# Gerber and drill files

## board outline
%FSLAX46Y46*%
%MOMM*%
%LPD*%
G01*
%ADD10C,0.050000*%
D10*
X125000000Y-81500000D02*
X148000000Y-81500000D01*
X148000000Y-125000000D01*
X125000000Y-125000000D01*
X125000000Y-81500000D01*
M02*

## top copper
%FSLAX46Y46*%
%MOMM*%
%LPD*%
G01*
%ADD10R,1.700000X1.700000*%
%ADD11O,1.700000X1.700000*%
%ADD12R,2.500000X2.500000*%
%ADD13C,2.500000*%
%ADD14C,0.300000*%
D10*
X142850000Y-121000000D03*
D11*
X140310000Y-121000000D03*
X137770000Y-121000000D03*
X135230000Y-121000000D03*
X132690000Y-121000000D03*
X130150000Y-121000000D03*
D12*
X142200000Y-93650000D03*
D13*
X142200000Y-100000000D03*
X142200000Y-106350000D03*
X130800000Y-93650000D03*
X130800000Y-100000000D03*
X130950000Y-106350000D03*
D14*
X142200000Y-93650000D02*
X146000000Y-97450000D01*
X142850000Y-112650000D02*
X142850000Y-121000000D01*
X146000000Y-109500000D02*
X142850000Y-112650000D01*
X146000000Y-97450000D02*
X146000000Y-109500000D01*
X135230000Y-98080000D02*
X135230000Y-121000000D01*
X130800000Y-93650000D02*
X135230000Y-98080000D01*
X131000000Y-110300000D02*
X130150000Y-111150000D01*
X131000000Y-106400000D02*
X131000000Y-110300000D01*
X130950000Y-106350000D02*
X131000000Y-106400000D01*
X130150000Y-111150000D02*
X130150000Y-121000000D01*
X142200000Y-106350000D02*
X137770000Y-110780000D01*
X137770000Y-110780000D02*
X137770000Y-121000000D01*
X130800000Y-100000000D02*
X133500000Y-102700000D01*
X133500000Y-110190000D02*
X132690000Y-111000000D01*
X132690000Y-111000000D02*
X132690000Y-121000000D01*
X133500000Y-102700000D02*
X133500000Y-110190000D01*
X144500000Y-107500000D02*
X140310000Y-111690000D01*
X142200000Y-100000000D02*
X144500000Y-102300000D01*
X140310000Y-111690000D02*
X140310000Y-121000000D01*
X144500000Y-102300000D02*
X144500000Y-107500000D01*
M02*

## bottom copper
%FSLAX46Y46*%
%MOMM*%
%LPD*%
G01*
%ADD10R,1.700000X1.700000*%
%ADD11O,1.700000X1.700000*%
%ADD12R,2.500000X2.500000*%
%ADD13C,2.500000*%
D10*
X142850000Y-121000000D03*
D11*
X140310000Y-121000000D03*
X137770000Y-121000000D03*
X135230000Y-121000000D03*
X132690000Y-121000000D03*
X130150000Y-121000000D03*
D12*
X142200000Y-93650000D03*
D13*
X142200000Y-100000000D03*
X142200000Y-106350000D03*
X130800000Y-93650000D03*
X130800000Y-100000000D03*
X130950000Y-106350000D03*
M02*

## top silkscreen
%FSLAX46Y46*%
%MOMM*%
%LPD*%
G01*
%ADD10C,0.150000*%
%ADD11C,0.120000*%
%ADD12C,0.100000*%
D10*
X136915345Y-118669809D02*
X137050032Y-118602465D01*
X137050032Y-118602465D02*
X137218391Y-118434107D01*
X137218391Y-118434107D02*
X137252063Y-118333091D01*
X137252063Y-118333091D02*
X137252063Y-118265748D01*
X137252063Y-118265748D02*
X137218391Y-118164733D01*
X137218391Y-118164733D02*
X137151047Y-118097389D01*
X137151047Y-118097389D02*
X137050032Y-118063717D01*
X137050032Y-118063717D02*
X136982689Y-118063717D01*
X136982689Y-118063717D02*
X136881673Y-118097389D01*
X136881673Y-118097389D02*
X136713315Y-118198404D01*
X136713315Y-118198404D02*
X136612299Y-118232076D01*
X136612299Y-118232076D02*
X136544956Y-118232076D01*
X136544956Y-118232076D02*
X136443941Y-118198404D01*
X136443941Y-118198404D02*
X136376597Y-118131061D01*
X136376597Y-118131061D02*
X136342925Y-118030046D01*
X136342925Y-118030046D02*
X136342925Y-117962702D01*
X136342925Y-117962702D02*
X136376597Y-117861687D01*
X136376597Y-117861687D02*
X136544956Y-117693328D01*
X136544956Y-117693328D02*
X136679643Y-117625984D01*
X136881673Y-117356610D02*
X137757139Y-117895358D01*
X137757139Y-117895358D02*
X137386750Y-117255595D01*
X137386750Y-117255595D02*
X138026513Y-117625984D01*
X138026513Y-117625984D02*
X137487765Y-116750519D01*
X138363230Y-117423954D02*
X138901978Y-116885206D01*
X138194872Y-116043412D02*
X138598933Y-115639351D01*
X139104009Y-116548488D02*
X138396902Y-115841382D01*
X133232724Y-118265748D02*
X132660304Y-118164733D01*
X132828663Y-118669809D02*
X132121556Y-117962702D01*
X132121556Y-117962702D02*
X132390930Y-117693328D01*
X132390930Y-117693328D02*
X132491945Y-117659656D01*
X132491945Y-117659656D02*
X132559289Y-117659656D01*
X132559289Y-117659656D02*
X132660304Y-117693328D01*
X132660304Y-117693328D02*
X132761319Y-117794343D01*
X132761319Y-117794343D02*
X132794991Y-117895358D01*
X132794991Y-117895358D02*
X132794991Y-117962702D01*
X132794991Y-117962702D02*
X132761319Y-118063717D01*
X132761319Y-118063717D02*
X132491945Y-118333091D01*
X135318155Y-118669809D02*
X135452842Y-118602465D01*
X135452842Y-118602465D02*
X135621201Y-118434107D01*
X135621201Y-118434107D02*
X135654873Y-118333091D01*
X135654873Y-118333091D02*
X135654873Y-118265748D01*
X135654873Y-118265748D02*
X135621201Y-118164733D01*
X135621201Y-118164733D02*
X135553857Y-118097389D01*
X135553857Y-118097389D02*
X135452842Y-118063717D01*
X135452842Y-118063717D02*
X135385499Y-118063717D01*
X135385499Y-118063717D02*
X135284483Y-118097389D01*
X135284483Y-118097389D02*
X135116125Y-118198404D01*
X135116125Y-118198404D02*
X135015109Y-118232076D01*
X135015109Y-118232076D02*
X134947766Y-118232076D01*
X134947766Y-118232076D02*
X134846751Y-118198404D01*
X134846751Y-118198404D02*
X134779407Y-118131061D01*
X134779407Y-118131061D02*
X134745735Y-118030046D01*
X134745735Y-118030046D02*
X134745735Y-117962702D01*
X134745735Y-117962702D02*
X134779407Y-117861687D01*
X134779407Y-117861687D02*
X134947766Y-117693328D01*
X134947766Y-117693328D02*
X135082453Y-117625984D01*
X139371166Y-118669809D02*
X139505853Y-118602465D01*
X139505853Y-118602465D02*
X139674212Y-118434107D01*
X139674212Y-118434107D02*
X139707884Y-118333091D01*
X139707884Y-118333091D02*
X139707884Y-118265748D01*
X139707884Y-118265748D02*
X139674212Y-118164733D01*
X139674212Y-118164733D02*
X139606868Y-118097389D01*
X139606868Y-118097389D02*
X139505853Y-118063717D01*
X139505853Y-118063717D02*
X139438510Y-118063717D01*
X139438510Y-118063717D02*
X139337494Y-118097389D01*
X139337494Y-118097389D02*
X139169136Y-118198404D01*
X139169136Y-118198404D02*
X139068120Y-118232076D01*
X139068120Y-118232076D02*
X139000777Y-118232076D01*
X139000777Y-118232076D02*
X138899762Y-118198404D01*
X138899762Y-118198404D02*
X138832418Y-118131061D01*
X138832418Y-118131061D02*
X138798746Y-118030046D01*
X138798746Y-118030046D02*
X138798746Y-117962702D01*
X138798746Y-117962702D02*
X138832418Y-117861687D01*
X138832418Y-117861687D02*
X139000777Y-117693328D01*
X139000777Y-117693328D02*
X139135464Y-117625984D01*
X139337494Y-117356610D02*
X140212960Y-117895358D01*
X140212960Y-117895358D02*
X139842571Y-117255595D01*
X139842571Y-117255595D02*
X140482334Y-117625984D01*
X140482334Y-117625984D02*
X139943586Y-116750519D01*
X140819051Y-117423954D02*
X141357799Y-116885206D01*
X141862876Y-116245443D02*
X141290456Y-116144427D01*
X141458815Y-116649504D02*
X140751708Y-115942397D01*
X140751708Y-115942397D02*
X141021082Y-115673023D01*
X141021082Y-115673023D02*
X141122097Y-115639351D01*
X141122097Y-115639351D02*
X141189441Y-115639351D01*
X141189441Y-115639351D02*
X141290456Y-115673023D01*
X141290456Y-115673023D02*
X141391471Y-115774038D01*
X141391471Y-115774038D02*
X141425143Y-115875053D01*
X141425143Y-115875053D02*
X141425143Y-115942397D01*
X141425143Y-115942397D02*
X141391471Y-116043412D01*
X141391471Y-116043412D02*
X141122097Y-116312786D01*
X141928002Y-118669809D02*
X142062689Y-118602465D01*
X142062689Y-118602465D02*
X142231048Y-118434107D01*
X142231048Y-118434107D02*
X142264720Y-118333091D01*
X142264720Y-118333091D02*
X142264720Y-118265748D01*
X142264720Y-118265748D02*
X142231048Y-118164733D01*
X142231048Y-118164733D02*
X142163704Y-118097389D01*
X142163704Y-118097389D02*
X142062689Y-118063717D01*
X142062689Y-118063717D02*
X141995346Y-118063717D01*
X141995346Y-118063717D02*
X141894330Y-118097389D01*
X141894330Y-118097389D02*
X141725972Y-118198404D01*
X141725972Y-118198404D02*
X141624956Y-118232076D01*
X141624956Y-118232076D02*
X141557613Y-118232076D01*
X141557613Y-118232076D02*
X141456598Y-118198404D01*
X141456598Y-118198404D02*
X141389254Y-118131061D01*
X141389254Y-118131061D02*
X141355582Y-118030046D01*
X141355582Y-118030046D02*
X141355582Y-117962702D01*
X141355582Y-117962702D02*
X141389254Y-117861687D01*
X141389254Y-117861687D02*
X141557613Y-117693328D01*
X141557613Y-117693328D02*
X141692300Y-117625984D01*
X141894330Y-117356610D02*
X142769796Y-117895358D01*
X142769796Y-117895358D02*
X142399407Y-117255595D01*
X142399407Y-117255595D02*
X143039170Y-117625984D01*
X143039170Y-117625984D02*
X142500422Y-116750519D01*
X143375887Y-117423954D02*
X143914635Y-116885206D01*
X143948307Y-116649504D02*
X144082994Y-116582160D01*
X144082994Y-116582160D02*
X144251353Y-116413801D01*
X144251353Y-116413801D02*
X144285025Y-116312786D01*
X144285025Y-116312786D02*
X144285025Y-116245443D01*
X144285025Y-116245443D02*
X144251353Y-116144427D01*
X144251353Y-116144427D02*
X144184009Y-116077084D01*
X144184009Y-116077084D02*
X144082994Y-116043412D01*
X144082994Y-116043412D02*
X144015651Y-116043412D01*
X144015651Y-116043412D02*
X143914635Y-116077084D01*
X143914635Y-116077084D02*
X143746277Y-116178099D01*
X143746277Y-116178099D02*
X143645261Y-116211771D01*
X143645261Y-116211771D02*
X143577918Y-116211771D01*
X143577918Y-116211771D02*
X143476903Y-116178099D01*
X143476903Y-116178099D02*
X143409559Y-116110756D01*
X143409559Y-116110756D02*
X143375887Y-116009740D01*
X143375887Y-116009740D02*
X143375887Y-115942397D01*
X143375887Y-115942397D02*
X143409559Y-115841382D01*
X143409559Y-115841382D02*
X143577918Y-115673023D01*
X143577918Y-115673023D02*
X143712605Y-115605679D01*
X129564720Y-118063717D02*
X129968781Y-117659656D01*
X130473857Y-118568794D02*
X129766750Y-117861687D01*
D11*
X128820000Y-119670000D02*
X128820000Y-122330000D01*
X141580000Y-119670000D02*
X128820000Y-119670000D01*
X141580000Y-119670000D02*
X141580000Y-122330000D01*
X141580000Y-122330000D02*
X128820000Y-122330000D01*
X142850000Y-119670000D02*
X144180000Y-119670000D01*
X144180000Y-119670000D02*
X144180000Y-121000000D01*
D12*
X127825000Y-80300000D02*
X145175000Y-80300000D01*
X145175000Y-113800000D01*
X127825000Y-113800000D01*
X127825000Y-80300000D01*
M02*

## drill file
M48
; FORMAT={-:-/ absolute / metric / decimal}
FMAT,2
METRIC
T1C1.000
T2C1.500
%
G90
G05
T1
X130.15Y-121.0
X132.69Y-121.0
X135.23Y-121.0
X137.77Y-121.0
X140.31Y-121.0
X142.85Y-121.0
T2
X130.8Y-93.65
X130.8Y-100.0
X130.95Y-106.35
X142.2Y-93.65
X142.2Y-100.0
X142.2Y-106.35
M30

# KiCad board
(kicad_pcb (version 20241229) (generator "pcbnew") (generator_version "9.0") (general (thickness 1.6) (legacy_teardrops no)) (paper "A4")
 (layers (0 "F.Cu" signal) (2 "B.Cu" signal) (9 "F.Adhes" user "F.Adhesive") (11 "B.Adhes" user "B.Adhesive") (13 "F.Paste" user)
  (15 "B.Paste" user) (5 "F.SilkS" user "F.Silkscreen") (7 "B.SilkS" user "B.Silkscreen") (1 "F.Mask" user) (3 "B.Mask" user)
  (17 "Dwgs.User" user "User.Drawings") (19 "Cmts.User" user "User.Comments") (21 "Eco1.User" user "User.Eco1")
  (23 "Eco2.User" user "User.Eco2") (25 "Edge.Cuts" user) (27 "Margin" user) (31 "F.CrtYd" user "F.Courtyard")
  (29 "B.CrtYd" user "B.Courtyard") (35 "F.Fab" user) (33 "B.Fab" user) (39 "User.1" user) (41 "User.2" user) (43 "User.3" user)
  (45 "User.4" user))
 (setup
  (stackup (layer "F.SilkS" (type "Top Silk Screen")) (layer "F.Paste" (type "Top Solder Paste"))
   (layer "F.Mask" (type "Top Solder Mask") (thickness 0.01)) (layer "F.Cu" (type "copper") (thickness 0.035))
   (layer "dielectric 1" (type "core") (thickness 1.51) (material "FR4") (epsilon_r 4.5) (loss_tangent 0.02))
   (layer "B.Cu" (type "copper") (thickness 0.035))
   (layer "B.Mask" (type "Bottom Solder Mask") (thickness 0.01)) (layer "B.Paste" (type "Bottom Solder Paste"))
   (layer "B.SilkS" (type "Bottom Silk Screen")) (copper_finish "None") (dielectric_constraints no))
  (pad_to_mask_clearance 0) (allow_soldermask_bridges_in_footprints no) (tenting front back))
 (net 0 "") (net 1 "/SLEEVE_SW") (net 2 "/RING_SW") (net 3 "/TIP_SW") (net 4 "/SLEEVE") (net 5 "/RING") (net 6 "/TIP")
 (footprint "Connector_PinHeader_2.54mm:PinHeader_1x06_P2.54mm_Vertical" (layer "F.Cu") (at 142.85 121 -90)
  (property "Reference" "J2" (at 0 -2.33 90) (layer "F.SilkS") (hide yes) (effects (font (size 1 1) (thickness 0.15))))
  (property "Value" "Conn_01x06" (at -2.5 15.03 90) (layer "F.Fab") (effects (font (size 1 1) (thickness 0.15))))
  (fp_line (start -1.33 14.03) (end 1.33 14.03) (stroke (width 0.12) (type solid)) (layer "F.SilkS"))
  (fp_line (start -1.33 1.27) (end -1.33 14.03) (stroke (width 0.12) (type solid)) (layer "F.SilkS"))
  (fp_line (start -1.33 1.27) (end 1.33 1.27) (stroke (width 0.12) (type solid)) (layer "F.SilkS"))
  (fp_line (start 1.33 1.27) (end 1.33 14.03) (stroke (width 0.12) (type solid)) (layer "F.SilkS"))
  (fp_line (start -1.33 0) (end -1.33 -1.33) (stroke (width 0.12) (type solid)) (layer "F.SilkS"))
  (fp_line (start -1.33 -1.33) (end 0 -1.33) (stroke (width 0.12) (type solid)) (layer "F.SilkS"))
  (pad "1" thru_hole rect (at 0 0 270) (size 1.7 1.7) (drill 1) (layers "*.Cu" "*.Mask") (remove_unused_layers no) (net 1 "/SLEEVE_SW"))
  (pad "2" thru_hole oval (at 0 2.54 270) (size 1.7 1.7) (drill 1) (layers "*.Cu" "*.Mask") (remove_unused_layers no) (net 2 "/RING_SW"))
  (pad "3" thru_hole oval (at 0 5.08 270) (size 1.7 1.7) (drill 1) (layers "*.Cu" "*.Mask") (remove_unused_layers no) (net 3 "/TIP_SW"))
  (pad "4" thru_hole oval (at 0 7.62 270) (size 1.7 1.7) (drill 1) (layers "*.Cu" "*.Mask") (remove_unused_layers no) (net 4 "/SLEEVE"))
  (pad "5" thru_hole oval (at 0 10.16 270) (size 1.7 1.7) (drill 1) (layers "*.Cu" "*.Mask") (remove_unused_layers no) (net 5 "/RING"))
  (pad "6" thru_hole oval (at 0 12.7 270) (size 1.7 1.7) (drill 1) (layers "*.Cu" "*.Mask") (remove_unused_layers no) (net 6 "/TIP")))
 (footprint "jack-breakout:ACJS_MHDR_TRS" (layer "F.Cu") (at 136.5 100 90)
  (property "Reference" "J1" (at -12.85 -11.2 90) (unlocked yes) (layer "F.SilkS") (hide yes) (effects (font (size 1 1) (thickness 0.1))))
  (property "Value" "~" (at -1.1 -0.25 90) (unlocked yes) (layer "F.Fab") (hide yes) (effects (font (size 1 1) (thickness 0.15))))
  (fp_rect (start -13.8 -8.675) (end 19.7 8.675) (stroke (width 0.1) (type solid)) (fill no) (layer "F.SilkS"))
  (pad "1" thru_hole rect (at 6.35 5.7 90) (size 2.5 2.5) (drill 1.5) (layers "*.Cu" "*.Mask") (remove_unused_layers no)
   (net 1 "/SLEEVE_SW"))
  (pad "2" thru_hole circle (at 0 5.7 90) (size 2.5 2.5) (drill 1.5) (layers "*.Cu" "*.Mask" "Eco2.User") (remove_unused_layers no)
   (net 2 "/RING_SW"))
  (pad "3" thru_hole circle (at -6.35 5.7 90) (size 2.5 2.5) (drill 1.5) (layers "*.Cu" "*.Mask") (remove_unused_layers no)
   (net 3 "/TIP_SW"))
  (pad "4" thru_hole circle (at 6.35 -5.7 90) (size 2.5 2.5) (drill 1.5) (layers "*.Cu" "*.Mask") (remove_unused_layers no)
   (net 4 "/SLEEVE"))
  (pad "5" thru_hole circle (at 0 -5.7 90) (size 2.5 2.5) (drill 1.5) (layers "*.Cu" "*.Mask") (remove_unused_layers no) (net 5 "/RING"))
  (pad "6" thru_hole circle (at -6.35 -5.55 90) (size 2.5 2.5) (drill 1.5) (layers "*.Cu" "*.Mask") (remove_unused_layers no) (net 6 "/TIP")))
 (gr_rect (start 125 81.5) (end 148 125) (stroke (width 0.05) (type default)) (fill no) (layer "Edge.Cuts"))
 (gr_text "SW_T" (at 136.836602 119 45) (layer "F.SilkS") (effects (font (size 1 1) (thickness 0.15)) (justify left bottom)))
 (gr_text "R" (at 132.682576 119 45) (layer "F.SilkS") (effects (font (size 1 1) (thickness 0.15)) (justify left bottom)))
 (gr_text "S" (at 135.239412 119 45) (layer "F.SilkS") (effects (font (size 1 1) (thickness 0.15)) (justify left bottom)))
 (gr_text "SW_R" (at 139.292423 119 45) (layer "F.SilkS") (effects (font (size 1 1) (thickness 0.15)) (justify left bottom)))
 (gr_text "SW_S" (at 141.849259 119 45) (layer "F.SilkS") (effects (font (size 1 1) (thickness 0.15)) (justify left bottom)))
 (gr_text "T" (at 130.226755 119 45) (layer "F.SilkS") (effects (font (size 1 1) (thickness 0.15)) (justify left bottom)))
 (segment (start 142.2 93.65) (end 146 97.45) (width 0.3) (layer "F.Cu") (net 1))
 (segment (start 142.85 112.65) (end 142.85 121) (width 0.3) (layer "F.Cu") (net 1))
 (segment (start 146 109.5) (end 142.85 112.65) (width 0.3) (layer "F.Cu") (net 1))
 (segment (start 146 97.45) (end 146 109.5) (width 0.3) (layer "F.Cu") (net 1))
 (segment (start 135.23 98.08) (end 135.23 121) (width 0.3) (layer "F.Cu") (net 4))
 (segment (start 130.8 93.65) (end 135.23 98.08) (width 0.3) (layer "F.Cu") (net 4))
 (segment (start 131 110.3) (end 130.15 111.15) (width 0.3) (layer "F.Cu") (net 6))
 (segment (start 131 106.4) (end 131 110.3) (width 0.3) (layer "F.Cu") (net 6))
 (segment (start 130.95 106.35) (end 131 106.4) (width 0.3) (layer "F.Cu") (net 6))
 (segment (start 130.15 111.15) (end 130.15 121) (width 0.3) (layer "F.Cu") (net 6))
 (segment (start 142.2 106.35) (end 137.77 110.78) (width 0.3) (layer "F.Cu") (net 3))
 (segment (start 137.77 110.78) (end 137.77 121) (width 0.3) (layer "F.Cu") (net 3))
 (segment (start 130.8 100) (end 133.5 102.7) (width 0.3) (layer "F.Cu") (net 5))
 (segment (start 133.5 110.19) (end 132.69 111) (width 0.3) (layer "F.Cu") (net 5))
 (segment (start 132.69 111) (end 132.69 121) (width 0.3) (layer "F.Cu") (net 5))
 (segment (start 133.5 102.7) (end 133.5 110.19) (width 0.3) (layer "F.Cu") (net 5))
 (segment (start 144.5 107.5) (end 140.31 111.69) (width 0.3) (layer "F.Cu") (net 2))
 (segment (start 142.2 100) (end 144.5 102.3) (width 0.3) (layer "F.Cu") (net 2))
 (segment (start 140.31 111.69) (end 140.31 121) (width 0.3) (layer "F.Cu") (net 2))
 (segment (start 144.5 102.3) (end 144.5 107.5) (width 0.3) (layer "F.Cu") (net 2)))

